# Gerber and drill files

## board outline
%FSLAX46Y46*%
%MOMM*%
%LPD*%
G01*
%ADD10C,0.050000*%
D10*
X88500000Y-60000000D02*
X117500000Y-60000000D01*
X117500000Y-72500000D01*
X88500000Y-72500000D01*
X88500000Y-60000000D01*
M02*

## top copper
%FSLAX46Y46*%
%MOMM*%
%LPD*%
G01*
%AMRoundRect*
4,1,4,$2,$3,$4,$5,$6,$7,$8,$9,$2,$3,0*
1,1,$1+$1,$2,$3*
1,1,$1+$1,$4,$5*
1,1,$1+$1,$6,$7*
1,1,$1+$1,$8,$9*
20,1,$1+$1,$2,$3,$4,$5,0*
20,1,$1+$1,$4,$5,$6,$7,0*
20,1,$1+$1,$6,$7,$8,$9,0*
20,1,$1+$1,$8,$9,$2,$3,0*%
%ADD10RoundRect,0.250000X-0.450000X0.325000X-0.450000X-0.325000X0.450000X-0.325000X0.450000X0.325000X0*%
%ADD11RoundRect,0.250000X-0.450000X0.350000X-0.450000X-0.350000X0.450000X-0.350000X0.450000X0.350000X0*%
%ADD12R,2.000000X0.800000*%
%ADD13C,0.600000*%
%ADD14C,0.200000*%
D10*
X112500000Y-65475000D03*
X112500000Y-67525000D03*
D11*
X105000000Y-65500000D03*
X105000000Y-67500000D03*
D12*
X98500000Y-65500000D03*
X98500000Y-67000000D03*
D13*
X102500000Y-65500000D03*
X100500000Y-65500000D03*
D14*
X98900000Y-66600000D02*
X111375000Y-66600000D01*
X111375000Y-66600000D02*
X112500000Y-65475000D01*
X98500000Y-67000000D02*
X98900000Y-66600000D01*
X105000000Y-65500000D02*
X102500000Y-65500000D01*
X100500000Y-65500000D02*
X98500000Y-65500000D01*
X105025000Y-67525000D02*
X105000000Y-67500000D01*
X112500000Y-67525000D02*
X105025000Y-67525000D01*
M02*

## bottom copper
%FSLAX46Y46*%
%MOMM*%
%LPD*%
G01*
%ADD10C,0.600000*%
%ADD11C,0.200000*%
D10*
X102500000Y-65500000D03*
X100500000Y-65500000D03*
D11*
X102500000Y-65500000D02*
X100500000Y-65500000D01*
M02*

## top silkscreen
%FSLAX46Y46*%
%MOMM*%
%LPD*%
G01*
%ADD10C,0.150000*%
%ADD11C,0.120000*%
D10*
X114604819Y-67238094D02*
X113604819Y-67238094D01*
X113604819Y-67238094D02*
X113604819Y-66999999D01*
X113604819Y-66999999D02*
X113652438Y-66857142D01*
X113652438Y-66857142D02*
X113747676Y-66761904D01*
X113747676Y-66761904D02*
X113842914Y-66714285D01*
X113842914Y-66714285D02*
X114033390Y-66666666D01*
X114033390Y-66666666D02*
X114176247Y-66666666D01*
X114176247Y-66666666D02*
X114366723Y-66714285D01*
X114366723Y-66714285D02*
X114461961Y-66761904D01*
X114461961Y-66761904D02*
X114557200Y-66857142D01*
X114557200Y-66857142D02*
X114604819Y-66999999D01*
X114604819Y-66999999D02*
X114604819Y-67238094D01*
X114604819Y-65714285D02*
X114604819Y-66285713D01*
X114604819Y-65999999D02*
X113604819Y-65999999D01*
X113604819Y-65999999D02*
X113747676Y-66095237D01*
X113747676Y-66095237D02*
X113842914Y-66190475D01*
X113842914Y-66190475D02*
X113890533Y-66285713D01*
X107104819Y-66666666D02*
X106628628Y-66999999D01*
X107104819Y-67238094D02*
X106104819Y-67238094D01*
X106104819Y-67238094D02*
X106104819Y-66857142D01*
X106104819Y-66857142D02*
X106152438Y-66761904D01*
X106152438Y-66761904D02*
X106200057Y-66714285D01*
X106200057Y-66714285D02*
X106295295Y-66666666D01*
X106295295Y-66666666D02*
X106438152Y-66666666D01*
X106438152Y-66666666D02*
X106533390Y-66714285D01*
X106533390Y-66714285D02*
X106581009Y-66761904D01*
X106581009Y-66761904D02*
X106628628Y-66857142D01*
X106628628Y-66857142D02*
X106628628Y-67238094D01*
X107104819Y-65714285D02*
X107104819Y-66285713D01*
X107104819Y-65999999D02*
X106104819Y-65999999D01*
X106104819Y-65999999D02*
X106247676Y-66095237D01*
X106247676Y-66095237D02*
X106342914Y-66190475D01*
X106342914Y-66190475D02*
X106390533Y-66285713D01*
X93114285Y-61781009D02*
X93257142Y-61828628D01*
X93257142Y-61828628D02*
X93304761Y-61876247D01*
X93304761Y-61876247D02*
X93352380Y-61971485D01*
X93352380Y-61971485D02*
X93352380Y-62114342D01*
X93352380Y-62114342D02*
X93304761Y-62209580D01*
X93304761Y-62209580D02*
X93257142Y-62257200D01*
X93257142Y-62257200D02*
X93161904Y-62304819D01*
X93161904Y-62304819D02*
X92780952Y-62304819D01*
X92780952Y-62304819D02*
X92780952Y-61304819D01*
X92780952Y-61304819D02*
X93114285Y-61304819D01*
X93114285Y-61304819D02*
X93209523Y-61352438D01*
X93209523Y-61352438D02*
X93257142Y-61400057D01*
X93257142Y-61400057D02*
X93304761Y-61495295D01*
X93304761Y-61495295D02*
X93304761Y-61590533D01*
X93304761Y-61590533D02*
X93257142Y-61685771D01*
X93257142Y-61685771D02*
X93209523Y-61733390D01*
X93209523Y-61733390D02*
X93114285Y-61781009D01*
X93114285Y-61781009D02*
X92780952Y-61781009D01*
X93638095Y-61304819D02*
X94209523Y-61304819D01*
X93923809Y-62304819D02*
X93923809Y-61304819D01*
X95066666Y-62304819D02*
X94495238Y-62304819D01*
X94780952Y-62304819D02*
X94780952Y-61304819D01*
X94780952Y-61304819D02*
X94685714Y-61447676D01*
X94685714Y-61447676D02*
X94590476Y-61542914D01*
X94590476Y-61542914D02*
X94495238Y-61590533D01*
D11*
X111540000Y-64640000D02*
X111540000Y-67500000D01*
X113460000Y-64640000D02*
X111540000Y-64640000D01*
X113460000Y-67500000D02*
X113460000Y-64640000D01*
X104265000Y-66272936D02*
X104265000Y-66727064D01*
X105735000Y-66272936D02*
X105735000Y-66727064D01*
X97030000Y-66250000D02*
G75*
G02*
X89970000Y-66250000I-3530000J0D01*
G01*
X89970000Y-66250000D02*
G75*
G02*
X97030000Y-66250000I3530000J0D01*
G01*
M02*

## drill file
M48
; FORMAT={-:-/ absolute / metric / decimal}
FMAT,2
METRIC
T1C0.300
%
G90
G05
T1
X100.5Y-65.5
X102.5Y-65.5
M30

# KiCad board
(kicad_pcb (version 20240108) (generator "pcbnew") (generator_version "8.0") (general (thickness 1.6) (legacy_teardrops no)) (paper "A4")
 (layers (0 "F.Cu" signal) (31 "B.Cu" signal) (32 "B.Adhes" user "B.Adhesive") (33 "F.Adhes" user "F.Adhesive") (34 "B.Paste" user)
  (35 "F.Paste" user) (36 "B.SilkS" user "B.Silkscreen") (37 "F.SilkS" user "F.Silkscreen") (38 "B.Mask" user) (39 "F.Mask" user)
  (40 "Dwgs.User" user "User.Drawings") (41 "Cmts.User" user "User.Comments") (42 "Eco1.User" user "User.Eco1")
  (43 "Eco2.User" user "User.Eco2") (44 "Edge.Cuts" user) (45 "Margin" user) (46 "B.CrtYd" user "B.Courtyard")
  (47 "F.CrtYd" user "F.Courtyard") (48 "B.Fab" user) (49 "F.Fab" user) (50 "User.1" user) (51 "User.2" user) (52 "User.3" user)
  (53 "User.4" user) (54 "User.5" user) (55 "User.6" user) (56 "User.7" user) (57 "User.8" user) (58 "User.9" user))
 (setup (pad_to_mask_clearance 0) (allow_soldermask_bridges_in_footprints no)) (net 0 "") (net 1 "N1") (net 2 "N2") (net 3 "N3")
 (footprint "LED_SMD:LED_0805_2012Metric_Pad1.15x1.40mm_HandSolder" (layer "F.Cu") (at 112.5 66.5 -90)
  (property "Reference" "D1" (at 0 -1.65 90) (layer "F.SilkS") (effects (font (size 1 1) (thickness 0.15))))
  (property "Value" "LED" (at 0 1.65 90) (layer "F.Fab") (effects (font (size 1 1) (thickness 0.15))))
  (fp_line (start -1.86 0.96) (end 1 0.96) (stroke (width 0.12) (type solid)) (layer "F.SilkS"))
  (fp_line (start -1.86 -0.96) (end -1.86 0.96) (stroke (width 0.12) (type solid)) (layer "F.SilkS"))
  (fp_line (start 1 -0.96) (end -1.86 -0.96) (stroke (width 0.12) (type solid)) (layer "F.SilkS"))
  (pad "1" smd roundrect (at -1.025 0 270) (size 1.15 1.4) (layers "F.Cu" "F.Paste" "F.Mask") (roundrect_rratio 0.217391) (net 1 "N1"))
  (pad "2" smd roundrect (at 1.025 0 270) (size 1.15 1.4) (layers "F.Cu" "F.Paste" "F.Mask") (roundrect_rratio 0.217391) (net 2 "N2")))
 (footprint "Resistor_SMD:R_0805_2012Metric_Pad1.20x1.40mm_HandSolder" (layer "F.Cu") (at 105 66.5 -90)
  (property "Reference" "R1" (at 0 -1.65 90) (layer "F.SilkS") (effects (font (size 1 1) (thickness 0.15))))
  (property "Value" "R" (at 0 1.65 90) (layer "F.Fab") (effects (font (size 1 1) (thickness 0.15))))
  (fp_line (start -0.227064 0.735) (end 0.227064 0.735) (stroke (width 0.12) (type solid)) (layer "F.SilkS"))
  (fp_line (start -0.227064 -0.735) (end 0.227064 -0.735) (stroke (width 0.12) (type solid)) (layer "F.SilkS"))
  (pad "1" smd roundrect (at -1 0 270) (size 1.2 1.4) (layers "F.Cu" "F.Paste" "F.Mask") (roundrect_rratio 0.208333) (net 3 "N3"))
  (pad "2" smd roundrect (at 1 0 270) (size 1.2 1.4) (layers "F.Cu" "F.Paste" "F.Mask") (roundrect_rratio 0.208333) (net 2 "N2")))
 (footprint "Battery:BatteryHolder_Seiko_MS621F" (layer "F.Cu") (at 98.5 66.25)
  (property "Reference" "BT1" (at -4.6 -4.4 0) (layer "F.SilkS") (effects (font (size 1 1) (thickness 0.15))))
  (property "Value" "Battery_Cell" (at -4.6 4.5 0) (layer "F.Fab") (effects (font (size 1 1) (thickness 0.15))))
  (fp_circle (center -5 0) (end -1.47 0) (stroke (width 0.12) (type solid)) (fill none) (layer "F.SilkS"))
  (pad "1" smd rect (at 0 -0.75) (size 2 0.8) (layers "F.Cu" "F.Paste" "F.Mask") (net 3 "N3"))
  (pad "2" smd rect (at 0 0.75) (size 2 0.8) (layers "F.Cu" "F.Paste" "F.Mask") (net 1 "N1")))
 (gr_rect (start 88.5 60) (end 117.5 72.5) (stroke (width 0.05) (type default)) (fill none) (layer "Edge.Cuts"))
 (segment (start 98.9 66.6) (end 111.375 66.6) (width 0.2) (layer "F.Cu") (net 1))
 (segment (start 111.375 66.6) (end 112.5 65.475) (width 0.2) (layer "F.Cu") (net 1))
 (segment (start 98.5 67) (end 98.9 66.6) (width 0.2) (layer "F.Cu") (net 1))
 (segment (start 105 65.5) (end 102.5 65.5) (width 0.2) (layer "F.Cu") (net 3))
 (segment (start 100.5 65.5) (end 98.5 65.5) (width 0.2) (layer "F.Cu") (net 3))
 (via (at 102.5 65.5) (size 0.6) (drill 0.3) (layers "F.Cu" "B.Cu") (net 3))
 (via (at 100.5 65.5) (size 0.6) (drill 0.3) (layers "F.Cu" "B.Cu") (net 3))
 (segment (start 102.5 65.5) (end 100.5 65.5) (width 0.2) (layer "B.Cu") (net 3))
 (segment (start 105.025 67.525) (end 105 67.5) (width 0.2) (layer "F.Cu") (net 2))
 (segment (start 112.5 67.525) (end 105.025 67.525) (width 0.2) (layer "F.Cu") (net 2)))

